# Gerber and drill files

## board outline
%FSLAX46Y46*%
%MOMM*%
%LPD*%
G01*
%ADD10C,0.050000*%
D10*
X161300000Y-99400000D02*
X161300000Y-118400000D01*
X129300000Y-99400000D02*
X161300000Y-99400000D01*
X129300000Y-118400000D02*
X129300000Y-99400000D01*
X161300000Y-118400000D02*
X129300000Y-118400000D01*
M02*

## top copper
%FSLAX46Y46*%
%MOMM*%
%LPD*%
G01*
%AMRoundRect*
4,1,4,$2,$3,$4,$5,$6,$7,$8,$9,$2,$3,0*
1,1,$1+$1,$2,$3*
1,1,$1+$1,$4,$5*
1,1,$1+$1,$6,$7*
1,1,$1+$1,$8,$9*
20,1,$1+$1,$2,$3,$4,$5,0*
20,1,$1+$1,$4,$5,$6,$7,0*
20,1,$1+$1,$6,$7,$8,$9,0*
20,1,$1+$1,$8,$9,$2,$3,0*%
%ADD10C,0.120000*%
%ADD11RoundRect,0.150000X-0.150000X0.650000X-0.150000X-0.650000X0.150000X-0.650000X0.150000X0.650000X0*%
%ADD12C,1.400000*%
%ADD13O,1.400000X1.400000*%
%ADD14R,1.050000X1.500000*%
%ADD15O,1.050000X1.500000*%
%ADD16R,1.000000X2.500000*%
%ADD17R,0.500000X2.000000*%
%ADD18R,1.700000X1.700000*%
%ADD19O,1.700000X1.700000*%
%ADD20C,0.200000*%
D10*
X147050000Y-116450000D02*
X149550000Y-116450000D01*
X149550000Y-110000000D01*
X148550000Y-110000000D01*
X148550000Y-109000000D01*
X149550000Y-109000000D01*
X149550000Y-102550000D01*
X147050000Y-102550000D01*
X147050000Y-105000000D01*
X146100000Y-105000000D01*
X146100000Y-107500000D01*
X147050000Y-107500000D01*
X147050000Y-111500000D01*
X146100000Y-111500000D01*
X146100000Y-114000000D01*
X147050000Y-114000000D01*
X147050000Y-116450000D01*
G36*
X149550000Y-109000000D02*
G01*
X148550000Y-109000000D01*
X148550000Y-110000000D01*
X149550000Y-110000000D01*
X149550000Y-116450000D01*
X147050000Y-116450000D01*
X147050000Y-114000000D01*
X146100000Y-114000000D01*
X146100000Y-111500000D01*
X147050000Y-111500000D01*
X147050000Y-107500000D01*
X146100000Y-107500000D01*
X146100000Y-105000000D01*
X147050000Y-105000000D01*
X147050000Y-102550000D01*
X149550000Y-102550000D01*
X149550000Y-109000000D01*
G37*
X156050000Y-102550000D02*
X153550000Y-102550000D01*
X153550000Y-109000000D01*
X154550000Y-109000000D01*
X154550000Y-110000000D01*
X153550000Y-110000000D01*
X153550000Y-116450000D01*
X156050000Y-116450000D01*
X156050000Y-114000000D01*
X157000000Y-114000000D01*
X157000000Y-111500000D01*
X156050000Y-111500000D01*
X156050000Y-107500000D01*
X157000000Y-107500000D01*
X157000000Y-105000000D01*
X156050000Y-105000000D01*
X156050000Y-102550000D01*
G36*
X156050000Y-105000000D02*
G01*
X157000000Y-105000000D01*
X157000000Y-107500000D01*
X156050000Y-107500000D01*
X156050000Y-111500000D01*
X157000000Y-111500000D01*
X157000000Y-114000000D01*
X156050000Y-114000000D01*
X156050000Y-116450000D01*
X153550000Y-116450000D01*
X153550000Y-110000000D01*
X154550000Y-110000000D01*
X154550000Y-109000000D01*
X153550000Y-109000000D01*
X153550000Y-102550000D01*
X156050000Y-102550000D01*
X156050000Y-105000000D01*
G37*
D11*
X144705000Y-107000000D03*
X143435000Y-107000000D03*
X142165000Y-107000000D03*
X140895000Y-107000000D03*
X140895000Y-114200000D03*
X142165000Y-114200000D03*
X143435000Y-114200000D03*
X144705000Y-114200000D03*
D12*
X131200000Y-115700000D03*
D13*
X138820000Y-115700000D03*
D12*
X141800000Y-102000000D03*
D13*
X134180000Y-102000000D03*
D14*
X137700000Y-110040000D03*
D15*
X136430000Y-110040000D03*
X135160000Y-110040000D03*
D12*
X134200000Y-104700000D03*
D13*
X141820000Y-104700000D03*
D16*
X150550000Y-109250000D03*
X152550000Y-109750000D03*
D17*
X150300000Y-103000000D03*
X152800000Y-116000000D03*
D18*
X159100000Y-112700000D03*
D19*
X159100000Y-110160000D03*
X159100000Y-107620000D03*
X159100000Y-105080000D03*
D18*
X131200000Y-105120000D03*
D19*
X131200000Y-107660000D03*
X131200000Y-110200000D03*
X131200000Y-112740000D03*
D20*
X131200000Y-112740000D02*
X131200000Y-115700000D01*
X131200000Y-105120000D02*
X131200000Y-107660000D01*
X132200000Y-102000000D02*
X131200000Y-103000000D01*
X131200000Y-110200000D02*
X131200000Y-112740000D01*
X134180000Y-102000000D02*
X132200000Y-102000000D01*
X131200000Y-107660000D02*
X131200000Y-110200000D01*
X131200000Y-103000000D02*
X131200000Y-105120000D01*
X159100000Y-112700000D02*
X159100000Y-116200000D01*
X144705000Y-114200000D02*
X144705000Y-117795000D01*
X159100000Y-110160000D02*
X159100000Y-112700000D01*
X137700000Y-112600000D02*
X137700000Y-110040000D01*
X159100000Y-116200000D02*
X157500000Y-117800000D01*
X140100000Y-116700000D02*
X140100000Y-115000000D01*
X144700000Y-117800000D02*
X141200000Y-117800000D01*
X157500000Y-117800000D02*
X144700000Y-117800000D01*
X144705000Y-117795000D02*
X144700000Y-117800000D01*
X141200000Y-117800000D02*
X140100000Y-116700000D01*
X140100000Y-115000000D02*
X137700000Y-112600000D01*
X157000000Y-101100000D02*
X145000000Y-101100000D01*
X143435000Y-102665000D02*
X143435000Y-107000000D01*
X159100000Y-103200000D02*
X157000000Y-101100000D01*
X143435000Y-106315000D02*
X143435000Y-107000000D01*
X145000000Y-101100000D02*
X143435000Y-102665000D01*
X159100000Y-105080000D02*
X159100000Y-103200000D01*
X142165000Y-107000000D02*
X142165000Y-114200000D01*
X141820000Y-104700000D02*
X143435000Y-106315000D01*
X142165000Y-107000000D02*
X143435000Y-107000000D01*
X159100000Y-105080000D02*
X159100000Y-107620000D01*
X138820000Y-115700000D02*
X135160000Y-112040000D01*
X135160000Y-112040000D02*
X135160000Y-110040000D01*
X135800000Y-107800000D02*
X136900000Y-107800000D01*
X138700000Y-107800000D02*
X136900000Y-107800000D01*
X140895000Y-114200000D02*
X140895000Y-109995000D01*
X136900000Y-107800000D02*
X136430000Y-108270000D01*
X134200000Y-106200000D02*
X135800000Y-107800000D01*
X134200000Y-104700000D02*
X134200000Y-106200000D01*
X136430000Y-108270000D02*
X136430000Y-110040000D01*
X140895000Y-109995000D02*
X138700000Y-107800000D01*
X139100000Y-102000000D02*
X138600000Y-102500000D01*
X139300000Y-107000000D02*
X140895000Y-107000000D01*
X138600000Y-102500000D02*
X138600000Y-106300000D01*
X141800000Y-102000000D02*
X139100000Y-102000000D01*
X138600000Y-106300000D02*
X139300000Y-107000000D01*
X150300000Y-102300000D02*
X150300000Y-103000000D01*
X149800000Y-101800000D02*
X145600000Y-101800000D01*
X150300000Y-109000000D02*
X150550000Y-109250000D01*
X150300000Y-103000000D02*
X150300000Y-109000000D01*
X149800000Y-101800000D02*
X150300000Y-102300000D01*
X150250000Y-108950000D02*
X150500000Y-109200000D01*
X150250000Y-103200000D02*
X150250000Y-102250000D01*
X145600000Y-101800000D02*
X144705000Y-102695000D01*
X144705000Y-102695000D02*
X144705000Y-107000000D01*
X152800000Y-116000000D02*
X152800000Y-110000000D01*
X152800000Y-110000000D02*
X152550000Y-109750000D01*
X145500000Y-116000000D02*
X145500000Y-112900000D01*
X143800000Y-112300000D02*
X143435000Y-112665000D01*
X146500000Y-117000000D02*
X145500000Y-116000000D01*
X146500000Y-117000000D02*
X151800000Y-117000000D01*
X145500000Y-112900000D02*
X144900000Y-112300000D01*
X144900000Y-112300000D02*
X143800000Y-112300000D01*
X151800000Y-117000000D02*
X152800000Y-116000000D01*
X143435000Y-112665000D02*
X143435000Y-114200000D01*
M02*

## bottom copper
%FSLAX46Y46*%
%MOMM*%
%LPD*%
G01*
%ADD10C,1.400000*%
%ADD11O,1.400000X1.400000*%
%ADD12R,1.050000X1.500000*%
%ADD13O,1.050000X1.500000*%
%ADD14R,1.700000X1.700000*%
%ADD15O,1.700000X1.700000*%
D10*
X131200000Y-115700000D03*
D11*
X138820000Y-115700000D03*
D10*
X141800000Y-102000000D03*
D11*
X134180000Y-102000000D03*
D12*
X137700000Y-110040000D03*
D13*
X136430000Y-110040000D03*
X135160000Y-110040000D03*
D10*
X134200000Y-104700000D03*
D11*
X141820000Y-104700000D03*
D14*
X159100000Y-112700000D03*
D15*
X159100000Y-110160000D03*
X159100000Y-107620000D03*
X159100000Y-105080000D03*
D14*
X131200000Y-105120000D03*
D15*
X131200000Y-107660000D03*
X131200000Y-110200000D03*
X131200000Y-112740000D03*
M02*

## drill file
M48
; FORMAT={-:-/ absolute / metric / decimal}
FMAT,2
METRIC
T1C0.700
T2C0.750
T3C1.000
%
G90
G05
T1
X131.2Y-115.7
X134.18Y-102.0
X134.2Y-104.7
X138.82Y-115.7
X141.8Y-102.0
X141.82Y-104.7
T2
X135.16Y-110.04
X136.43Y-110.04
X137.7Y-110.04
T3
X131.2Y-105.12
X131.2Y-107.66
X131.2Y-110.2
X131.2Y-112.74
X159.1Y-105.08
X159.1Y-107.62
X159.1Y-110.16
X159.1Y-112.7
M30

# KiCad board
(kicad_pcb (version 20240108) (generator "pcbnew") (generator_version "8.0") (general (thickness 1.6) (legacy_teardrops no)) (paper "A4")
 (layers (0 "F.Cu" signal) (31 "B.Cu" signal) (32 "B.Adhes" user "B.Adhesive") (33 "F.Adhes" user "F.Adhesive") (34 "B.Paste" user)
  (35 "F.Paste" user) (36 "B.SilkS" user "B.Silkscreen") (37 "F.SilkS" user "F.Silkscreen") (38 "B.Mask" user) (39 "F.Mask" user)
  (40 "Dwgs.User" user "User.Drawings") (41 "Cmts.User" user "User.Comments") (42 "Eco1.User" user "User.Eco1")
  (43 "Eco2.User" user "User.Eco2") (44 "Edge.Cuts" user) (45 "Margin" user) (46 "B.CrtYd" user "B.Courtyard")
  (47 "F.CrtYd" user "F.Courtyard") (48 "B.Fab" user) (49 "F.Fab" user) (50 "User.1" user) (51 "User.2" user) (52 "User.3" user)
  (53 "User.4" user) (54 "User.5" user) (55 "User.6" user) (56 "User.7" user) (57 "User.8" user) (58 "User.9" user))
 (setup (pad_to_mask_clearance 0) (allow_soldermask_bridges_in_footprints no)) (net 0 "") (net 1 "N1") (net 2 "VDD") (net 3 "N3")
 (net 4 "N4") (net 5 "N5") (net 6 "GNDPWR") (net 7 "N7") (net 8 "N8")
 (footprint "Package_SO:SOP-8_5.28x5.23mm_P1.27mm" (layer "F.Cu") (at 142.8 110.6 -90)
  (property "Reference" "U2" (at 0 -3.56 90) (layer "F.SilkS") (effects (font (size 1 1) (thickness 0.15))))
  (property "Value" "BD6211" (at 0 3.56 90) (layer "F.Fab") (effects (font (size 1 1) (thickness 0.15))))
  (pad "1" smd roundrect (at -3.6 -1.905 270) (size 1.6 0.6) (layers "F.Cu" "F.Paste" "F.Mask") (roundrect_rratio 0.25) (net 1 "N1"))
  (pad "2" smd roundrect (at -3.6 -0.635 270) (size 1.6 0.6) (layers "F.Cu" "F.Paste" "F.Mask") (roundrect_rratio 0.25) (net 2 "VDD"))
  (pad "3" smd roundrect (at -3.6 0.635 270) (size 1.6 0.6) (layers "F.Cu" "F.Paste" "F.Mask") (roundrect_rratio 0.25) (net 2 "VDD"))
  (pad "4" smd roundrect (at -3.6 1.905 270) (size 1.6 0.6) (layers "F.Cu" "F.Paste" "F.Mask") (roundrect_rratio 0.25) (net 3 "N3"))
  (pad "5" smd roundrect (at 3.6 1.905 270) (size 1.6 0.6) (layers "F.Cu" "F.Paste" "F.Mask") (roundrect_rratio 0.25) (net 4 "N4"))
  (pad "6" smd roundrect (at 3.6 0.635 270) (size 1.6 0.6) (layers "F.Cu" "F.Paste" "F.Mask") (roundrect_rratio 0.25) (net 2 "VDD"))
  (pad "7" smd roundrect (at 3.6 -0.635 270) (size 1.6 0.6) (layers "F.Cu" "F.Paste" "F.Mask") (roundrect_rratio 0.25) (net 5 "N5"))
  (pad "8" smd roundrect (at 3.6 -1.905 270) (size 1.6 0.6) (layers "F.Cu" "F.Paste" "F.Mask") (roundrect_rratio 0.25) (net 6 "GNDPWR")))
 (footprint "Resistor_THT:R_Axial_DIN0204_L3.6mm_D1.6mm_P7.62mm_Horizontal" (layer "F.Cu") (at 131.2 115.7)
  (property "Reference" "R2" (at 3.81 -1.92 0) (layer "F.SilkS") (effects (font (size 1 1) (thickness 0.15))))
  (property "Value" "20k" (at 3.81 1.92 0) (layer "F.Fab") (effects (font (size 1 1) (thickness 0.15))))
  (pad "1" thru_hole circle (at 0 0) (size 1.4 1.4) (drill 0.7) (layers "*.Cu" "*.Mask") (remove_unused_layers no) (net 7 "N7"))
  (pad "2" thru_hole oval (at 7.62 0) (size 1.4 1.4) (drill 0.7) (layers "*.Cu" "*.Mask") (remove_unused_layers no) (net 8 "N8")))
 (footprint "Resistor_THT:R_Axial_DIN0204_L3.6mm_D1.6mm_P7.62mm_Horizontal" (layer "F.Cu") (at 141.8 102 180)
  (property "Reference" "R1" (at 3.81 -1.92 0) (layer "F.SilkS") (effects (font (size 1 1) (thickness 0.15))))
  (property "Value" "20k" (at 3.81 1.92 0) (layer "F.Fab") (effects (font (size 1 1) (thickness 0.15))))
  (pad "1" thru_hole circle (at 0 0 180) (size 1.4 1.4) (drill 0.7) (layers "*.Cu" "*.Mask") (remove_unused_layers no) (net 3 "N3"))
  (pad "2" thru_hole oval (at 7.62 0 180) (size 1.4 1.4) (drill 0.7) (layers "*.Cu" "*.Mask") (remove_unused_layers no) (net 7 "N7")))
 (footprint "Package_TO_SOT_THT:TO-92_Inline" (layer "F.Cu") (at 137.7 110.04 180)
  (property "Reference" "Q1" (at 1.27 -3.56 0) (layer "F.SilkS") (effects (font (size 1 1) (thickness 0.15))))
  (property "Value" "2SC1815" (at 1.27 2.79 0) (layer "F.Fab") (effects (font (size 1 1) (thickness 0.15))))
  (pad "1" thru_hole rect (at 0 0 180) (size 1.05 1.5) (drill 0.75) (layers "*.Cu" "*.Mask") (remove_unused_layers no) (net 6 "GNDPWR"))
  (pad "2" thru_hole oval (at 1.27 0 180) (size 1.05 1.5) (drill 0.75) (layers "*.Cu" "*.Mask") (remove_unused_layers no) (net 4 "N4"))
  (pad "3" thru_hole oval (at 2.54 0 180) (size 1.05 1.5) (drill 0.75) (layers "*.Cu" "*.Mask") (remove_unused_layers no) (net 8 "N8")))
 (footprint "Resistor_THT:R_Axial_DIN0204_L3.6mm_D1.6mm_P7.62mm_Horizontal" (layer "F.Cu") (at 134.2 104.7)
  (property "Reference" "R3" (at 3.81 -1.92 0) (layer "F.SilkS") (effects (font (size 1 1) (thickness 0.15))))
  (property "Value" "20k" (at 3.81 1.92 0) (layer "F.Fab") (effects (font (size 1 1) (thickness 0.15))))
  (pad "1" thru_hole circle (at 0 0) (size 1.4 1.4) (drill 0.7) (layers "*.Cu" "*.Mask") (remove_unused_layers no) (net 4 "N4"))
  (pad "2" thru_hole oval (at 7.62 0) (size 1.4 1.4) (drill 0.7) (layers "*.Cu" "*.Mask") (remove_unused_layers no) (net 2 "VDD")))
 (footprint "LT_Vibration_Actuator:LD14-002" (layer "F.Cu") (at 151.55 109.5)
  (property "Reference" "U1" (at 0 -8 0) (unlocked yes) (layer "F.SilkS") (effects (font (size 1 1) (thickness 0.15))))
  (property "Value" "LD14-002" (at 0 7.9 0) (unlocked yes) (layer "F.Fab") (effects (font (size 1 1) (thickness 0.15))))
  (fp_poly
   (pts (xy -4.5 6.95) (xy -2 6.95) (xy -2 0.5) (xy -3 0.5) (xy -3 -0.5) (xy -2 -0.5) (xy -2 -6.95) (xy -4.5 -6.95) (xy -4.5 -4.5)
    (xy -5.45 -4.5) (xy -5.45 -2) (xy -4.5 -2) (xy -4.5 2) (xy -5.45 2) (xy -5.45 4.5) (xy -4.5 4.5))
   (stroke (width 0.12) (type solid)) (fill solid) (layer "F.Cu"))
  (fp_poly
   (pts (xy 4.5 -6.95) (xy 2 -6.95) (xy 2 -0.5) (xy 3 -0.5) (xy 3 0.5) (xy 2 0.5) (xy 2 6.95) (xy 4.5 6.95) (xy 4.5 4.5) (xy 5.45 4.5)
    (xy 5.45 2) (xy 4.5 2) (xy 4.5 -2) (xy 5.45 -2) (xy 5.45 -4.5) (xy 4.5 -4.5))
   (stroke (width 0.12) (type solid)) (fill solid) (layer "F.Cu"))
  (pad "1" smd rect (at -1 -0.25) (size 1 2.5) (layers "F.Cu" "F.Paste" "F.Mask") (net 1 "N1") (thermal_bridge_angle 45))
  (pad "2" smd rect (at 1 0.25) (size 1 2.5) (layers "F.Cu" "F.Paste" "F.Mask") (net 5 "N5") (thermal_bridge_angle 45))
  (pad "3" smd rect (at -1.25 -6.5) (size 0.5 2) (layers "F.Cu" "F.Paste" "F.Mask") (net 1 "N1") (thermal_bridge_angle 45))
  (pad "4" smd rect (at 1.25 6.5) (size 0.5 2) (layers "F.Cu" "F.Paste" "F.Mask") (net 5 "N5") (thermal_bridge_angle 45)))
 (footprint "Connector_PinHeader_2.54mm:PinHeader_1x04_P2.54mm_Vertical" (layer "B.Cu") (at 159.1 112.7)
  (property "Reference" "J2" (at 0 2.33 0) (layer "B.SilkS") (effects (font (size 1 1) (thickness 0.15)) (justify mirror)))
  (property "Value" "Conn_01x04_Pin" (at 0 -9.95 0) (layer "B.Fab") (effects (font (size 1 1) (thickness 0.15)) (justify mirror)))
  (pad "1" thru_hole rect (at 0 0) (size 1.7 1.7) (drill 1) (layers "*.Cu" "*.Mask") (remove_unused_layers no) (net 6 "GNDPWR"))
  (pad "2" thru_hole oval (at 0 -2.54) (size 1.7 1.7) (drill 1) (layers "*.Cu" "*.Mask") (remove_unused_layers no) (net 6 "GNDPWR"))
  (pad "3" thru_hole oval (at 0 -5.08) (size 1.7 1.7) (drill 1) (layers "*.Cu" "*.Mask") (remove_unused_layers no) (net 2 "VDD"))
  (pad "4" thru_hole oval (at 0 -7.62) (size 1.7 1.7) (drill 1) (layers "*.Cu" "*.Mask") (remove_unused_layers no) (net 2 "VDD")))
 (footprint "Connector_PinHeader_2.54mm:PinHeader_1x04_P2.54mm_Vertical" (layer "B.Cu") (at 131.2 105.12 180)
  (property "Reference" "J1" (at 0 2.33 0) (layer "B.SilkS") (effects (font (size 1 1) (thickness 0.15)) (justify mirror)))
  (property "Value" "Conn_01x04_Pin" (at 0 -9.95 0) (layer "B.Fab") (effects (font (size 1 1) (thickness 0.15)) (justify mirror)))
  (pad "1" thru_hole rect (at 0 0 180) (size 1.7 1.7) (drill 1) (layers "*.Cu" "*.Mask") (remove_unused_layers no) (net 7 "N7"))
  (pad "2" thru_hole oval (at 0 -2.54 180) (size 1.7 1.7) (drill 1) (layers "*.Cu" "*.Mask") (remove_unused_layers no) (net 7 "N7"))
  (pad "3" thru_hole oval (at 0 -5.08 180) (size 1.7 1.7) (drill 1) (layers "*.Cu" "*.Mask") (remove_unused_layers no) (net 7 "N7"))
  (pad "4" thru_hole oval (at 0 -7.62 180) (size 1.7 1.7) (drill 1) (layers "*.Cu" "*.Mask") (remove_unused_layers no) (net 7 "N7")))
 (gr_line (start 161.3 99.4) (end 161.3 118.4) (stroke (width 0.05) (type default)) (layer "Edge.Cuts"))
 (gr_line (start 129.3 99.4) (end 161.3 99.4) (stroke (width 0.05) (type default)) (layer "Edge.Cuts"))
 (gr_line (start 129.3 118.4) (end 129.3 99.4) (stroke (width 0.05) (type default)) (layer "Edge.Cuts"))
 (gr_line (start 161.3 118.4) (end 129.3 118.4) (stroke (width 0.05) (type default)) (layer "Edge.Cuts"))
 (segment (start 131.2 112.74) (end 131.2 115.7) (width 0.2) (layer "F.Cu") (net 7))
 (segment (start 131.2 105.12) (end 131.2 107.66) (width 0.2) (layer "F.Cu") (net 7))
 (segment (start 132.2 102) (end 131.2 103) (width 0.2) (layer "F.Cu") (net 7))
 (segment (start 131.2 110.2) (end 131.2 112.74) (width 0.2) (layer "F.Cu") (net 7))
 (segment (start 134.18 102) (end 132.2 102) (width 0.2) (layer "F.Cu") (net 7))
 (segment (start 131.2 107.66) (end 131.2 110.2) (width 0.2) (layer "F.Cu") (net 7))
 (segment (start 131.2 103) (end 131.2 105.12) (width 0.2) (layer "F.Cu") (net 7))
 (segment (start 159.1 112.7) (end 159.1 116.2) (width 0.2) (layer "F.Cu") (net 6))
 (segment (start 144.705 114.2) (end 144.705 117.795) (width 0.2) (layer "F.Cu") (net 6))
 (segment (start 159.1 110.16) (end 159.1 112.7) (width 0.2) (layer "F.Cu") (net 6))
 (segment (start 137.7 112.6) (end 137.7 110.04) (width 0.2) (layer "F.Cu") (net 6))
 (segment (start 159.1 116.2) (end 157.5 117.8) (width 0.2) (layer "F.Cu") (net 6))
 (segment (start 140.1 116.7) (end 140.1 115) (width 0.2) (layer "F.Cu") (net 6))
 (segment (start 144.7 117.8) (end 141.2 117.8) (width 0.2) (layer "F.Cu") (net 6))
 (segment (start 157.5 117.8) (end 144.7 117.8) (width 0.2) (layer "F.Cu") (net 6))
 (segment (start 144.705 117.795) (end 144.7 117.8) (width 0.2) (layer "F.Cu") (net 6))
 (segment (start 141.2 117.8) (end 140.1 116.7) (width 0.2) (layer "F.Cu") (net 6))
 (segment (start 140.1 115) (end 137.7 112.6) (width 0.2) (layer "F.Cu") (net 6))
 (segment (start 157 101.1) (end 145 101.1) (width 0.2) (layer "F.Cu") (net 2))
 (segment (start 143.435 102.665) (end 143.435 107) (width 0.2) (layer "F.Cu") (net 2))
 (segment (start 159.1 103.2) (end 157 101.1) (width 0.2) (layer "F.Cu") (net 2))
 (segment (start 143.435 106.315) (end 143.435 107) (width 0.2) (layer "F.Cu") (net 2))
 (segment (start 145 101.1) (end 143.435 102.665) (width 0.2) (layer "F.Cu") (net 2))
 (segment (start 159.1 105.08) (end 159.1 103.2) (width 0.2) (layer "F.Cu") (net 2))
 (segment (start 142.165 107) (end 142.165 114.2) (width 0.2) (layer "F.Cu") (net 2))
 (segment (start 141.82 104.7) (end 143.435 106.315) (width 0.2) (layer "F.Cu") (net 2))
 (segment (start 142.165 107) (end 143.435 107) (width 0.2) (layer "F.Cu") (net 2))
 (segment (start 159.1 105.08) (end 159.1 107.62) (width 0.2) (layer "F.Cu") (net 2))
 (segment (start 138.82 115.7) (end 135.16 112.04) (width 0.2) (layer "F.Cu") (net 8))
 (segment (start 135.16 112.04) (end 135.16 110.04) (width 0.2) (layer "F.Cu") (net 8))
 (segment (start 135.8 107.8) (end 136.9 107.8) (width 0.2) (layer "F.Cu") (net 4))
 (segment (start 138.7 107.8) (end 136.9 107.8) (width 0.2) (layer "F.Cu") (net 4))
 (segment (start 140.895 114.2) (end 140.895 109.995) (width 0.2) (layer "F.Cu") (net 4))
 (segment (start 136.9 107.8) (end 136.43 108.27) (width 0.2) (layer "F.Cu") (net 4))
 (segment (start 134.2 106.2) (end 135.8 107.8) (width 0.2) (layer "F.Cu") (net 4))
 (segment (start 134.2 104.7) (end 134.2 106.2) (width 0.2) (layer "F.Cu") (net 4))
 (segment (start 136.43 108.27) (end 136.43 110.04) (width 0.2) (layer "F.Cu") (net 4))
 (segment (start 140.895 109.995) (end 138.7 107.8) (width 0.2) (layer "F.Cu") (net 4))
 (segment (start 139.1 102) (end 138.6 102.5) (width 0.2) (layer "F.Cu") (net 3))
 (segment (start 139.3 107) (end 140.895 107) (width 0.2) (layer "F.Cu") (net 3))
 (segment (start 138.6 102.5) (end 138.6 106.3) (width 0.2) (layer "F.Cu") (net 3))
 (segment (start 141.8 102) (end 139.1 102) (width 0.2) (layer "F.Cu") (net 3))
 (segment (start 138.6 106.3) (end 139.3 107) (width 0.2) (layer "F.Cu") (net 3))
 (segment (start 150.3 102.3) (end 150.3 103) (width 0.2) (layer "F.Cu") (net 1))
 (segment (start 149.8 101.8) (end 145.6 101.8) (width 0.2) (layer "F.Cu") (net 1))
 (segment (start 150.3 109) (end 150.55 109.25) (width 0.2) (layer "F.Cu") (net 1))
 (segment (start 150.3 103) (end 150.3 109) (width 0.2) (layer "F.Cu") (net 1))
 (segment (start 149.8 101.8) (end 150.3 102.3) (width 0.2) (layer "F.Cu") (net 1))
 (segment (start 150.25 108.95) (end 150.5 109.2) (width 0.2) (layer "F.Cu") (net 1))
 (segment (start 150.25 103.2) (end 150.25 102.25) (width 0.2) (layer "F.Cu") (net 1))
 (segment (start 145.6 101.8) (end 144.705 102.695) (width 0.2) (layer "F.Cu") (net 1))
 (segment (start 144.705 102.695) (end 144.705 107) (width 0.2) (layer "F.Cu") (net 1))
 (segment (start 152.8 116) (end 152.8 110) (width 0.2) (layer "F.Cu") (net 5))
 (segment (start 152.8 110) (end 152.55 109.75) (width 0.2) (layer "F.Cu") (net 5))
 (segment (start 145.5 116) (end 145.5 112.9) (width 0.2) (layer "F.Cu") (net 5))
 (segment (start 143.8 112.3) (end 143.435 112.665) (width 0.2) (layer "F.Cu") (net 5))
 (segment (start 146.5 117) (end 145.5 116) (width 0.2) (layer "F.Cu") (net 5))
 (segment (start 146.5 117) (end 151.8 117) (width 0.2) (layer "F.Cu") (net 5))
 (segment (start 145.5 112.9) (end 144.9 112.3) (width 0.2) (layer "F.Cu") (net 5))
 (segment (start 144.9 112.3) (end 143.8 112.3) (width 0.2) (layer "F.Cu") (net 5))
 (segment (start 151.8 117) (end 152.8 116) (width 0.2) (layer "F.Cu") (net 5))
 (segment (start 143.435 112.665) (end 143.435 114.2) (width 0.2) (layer "F.Cu") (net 5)))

